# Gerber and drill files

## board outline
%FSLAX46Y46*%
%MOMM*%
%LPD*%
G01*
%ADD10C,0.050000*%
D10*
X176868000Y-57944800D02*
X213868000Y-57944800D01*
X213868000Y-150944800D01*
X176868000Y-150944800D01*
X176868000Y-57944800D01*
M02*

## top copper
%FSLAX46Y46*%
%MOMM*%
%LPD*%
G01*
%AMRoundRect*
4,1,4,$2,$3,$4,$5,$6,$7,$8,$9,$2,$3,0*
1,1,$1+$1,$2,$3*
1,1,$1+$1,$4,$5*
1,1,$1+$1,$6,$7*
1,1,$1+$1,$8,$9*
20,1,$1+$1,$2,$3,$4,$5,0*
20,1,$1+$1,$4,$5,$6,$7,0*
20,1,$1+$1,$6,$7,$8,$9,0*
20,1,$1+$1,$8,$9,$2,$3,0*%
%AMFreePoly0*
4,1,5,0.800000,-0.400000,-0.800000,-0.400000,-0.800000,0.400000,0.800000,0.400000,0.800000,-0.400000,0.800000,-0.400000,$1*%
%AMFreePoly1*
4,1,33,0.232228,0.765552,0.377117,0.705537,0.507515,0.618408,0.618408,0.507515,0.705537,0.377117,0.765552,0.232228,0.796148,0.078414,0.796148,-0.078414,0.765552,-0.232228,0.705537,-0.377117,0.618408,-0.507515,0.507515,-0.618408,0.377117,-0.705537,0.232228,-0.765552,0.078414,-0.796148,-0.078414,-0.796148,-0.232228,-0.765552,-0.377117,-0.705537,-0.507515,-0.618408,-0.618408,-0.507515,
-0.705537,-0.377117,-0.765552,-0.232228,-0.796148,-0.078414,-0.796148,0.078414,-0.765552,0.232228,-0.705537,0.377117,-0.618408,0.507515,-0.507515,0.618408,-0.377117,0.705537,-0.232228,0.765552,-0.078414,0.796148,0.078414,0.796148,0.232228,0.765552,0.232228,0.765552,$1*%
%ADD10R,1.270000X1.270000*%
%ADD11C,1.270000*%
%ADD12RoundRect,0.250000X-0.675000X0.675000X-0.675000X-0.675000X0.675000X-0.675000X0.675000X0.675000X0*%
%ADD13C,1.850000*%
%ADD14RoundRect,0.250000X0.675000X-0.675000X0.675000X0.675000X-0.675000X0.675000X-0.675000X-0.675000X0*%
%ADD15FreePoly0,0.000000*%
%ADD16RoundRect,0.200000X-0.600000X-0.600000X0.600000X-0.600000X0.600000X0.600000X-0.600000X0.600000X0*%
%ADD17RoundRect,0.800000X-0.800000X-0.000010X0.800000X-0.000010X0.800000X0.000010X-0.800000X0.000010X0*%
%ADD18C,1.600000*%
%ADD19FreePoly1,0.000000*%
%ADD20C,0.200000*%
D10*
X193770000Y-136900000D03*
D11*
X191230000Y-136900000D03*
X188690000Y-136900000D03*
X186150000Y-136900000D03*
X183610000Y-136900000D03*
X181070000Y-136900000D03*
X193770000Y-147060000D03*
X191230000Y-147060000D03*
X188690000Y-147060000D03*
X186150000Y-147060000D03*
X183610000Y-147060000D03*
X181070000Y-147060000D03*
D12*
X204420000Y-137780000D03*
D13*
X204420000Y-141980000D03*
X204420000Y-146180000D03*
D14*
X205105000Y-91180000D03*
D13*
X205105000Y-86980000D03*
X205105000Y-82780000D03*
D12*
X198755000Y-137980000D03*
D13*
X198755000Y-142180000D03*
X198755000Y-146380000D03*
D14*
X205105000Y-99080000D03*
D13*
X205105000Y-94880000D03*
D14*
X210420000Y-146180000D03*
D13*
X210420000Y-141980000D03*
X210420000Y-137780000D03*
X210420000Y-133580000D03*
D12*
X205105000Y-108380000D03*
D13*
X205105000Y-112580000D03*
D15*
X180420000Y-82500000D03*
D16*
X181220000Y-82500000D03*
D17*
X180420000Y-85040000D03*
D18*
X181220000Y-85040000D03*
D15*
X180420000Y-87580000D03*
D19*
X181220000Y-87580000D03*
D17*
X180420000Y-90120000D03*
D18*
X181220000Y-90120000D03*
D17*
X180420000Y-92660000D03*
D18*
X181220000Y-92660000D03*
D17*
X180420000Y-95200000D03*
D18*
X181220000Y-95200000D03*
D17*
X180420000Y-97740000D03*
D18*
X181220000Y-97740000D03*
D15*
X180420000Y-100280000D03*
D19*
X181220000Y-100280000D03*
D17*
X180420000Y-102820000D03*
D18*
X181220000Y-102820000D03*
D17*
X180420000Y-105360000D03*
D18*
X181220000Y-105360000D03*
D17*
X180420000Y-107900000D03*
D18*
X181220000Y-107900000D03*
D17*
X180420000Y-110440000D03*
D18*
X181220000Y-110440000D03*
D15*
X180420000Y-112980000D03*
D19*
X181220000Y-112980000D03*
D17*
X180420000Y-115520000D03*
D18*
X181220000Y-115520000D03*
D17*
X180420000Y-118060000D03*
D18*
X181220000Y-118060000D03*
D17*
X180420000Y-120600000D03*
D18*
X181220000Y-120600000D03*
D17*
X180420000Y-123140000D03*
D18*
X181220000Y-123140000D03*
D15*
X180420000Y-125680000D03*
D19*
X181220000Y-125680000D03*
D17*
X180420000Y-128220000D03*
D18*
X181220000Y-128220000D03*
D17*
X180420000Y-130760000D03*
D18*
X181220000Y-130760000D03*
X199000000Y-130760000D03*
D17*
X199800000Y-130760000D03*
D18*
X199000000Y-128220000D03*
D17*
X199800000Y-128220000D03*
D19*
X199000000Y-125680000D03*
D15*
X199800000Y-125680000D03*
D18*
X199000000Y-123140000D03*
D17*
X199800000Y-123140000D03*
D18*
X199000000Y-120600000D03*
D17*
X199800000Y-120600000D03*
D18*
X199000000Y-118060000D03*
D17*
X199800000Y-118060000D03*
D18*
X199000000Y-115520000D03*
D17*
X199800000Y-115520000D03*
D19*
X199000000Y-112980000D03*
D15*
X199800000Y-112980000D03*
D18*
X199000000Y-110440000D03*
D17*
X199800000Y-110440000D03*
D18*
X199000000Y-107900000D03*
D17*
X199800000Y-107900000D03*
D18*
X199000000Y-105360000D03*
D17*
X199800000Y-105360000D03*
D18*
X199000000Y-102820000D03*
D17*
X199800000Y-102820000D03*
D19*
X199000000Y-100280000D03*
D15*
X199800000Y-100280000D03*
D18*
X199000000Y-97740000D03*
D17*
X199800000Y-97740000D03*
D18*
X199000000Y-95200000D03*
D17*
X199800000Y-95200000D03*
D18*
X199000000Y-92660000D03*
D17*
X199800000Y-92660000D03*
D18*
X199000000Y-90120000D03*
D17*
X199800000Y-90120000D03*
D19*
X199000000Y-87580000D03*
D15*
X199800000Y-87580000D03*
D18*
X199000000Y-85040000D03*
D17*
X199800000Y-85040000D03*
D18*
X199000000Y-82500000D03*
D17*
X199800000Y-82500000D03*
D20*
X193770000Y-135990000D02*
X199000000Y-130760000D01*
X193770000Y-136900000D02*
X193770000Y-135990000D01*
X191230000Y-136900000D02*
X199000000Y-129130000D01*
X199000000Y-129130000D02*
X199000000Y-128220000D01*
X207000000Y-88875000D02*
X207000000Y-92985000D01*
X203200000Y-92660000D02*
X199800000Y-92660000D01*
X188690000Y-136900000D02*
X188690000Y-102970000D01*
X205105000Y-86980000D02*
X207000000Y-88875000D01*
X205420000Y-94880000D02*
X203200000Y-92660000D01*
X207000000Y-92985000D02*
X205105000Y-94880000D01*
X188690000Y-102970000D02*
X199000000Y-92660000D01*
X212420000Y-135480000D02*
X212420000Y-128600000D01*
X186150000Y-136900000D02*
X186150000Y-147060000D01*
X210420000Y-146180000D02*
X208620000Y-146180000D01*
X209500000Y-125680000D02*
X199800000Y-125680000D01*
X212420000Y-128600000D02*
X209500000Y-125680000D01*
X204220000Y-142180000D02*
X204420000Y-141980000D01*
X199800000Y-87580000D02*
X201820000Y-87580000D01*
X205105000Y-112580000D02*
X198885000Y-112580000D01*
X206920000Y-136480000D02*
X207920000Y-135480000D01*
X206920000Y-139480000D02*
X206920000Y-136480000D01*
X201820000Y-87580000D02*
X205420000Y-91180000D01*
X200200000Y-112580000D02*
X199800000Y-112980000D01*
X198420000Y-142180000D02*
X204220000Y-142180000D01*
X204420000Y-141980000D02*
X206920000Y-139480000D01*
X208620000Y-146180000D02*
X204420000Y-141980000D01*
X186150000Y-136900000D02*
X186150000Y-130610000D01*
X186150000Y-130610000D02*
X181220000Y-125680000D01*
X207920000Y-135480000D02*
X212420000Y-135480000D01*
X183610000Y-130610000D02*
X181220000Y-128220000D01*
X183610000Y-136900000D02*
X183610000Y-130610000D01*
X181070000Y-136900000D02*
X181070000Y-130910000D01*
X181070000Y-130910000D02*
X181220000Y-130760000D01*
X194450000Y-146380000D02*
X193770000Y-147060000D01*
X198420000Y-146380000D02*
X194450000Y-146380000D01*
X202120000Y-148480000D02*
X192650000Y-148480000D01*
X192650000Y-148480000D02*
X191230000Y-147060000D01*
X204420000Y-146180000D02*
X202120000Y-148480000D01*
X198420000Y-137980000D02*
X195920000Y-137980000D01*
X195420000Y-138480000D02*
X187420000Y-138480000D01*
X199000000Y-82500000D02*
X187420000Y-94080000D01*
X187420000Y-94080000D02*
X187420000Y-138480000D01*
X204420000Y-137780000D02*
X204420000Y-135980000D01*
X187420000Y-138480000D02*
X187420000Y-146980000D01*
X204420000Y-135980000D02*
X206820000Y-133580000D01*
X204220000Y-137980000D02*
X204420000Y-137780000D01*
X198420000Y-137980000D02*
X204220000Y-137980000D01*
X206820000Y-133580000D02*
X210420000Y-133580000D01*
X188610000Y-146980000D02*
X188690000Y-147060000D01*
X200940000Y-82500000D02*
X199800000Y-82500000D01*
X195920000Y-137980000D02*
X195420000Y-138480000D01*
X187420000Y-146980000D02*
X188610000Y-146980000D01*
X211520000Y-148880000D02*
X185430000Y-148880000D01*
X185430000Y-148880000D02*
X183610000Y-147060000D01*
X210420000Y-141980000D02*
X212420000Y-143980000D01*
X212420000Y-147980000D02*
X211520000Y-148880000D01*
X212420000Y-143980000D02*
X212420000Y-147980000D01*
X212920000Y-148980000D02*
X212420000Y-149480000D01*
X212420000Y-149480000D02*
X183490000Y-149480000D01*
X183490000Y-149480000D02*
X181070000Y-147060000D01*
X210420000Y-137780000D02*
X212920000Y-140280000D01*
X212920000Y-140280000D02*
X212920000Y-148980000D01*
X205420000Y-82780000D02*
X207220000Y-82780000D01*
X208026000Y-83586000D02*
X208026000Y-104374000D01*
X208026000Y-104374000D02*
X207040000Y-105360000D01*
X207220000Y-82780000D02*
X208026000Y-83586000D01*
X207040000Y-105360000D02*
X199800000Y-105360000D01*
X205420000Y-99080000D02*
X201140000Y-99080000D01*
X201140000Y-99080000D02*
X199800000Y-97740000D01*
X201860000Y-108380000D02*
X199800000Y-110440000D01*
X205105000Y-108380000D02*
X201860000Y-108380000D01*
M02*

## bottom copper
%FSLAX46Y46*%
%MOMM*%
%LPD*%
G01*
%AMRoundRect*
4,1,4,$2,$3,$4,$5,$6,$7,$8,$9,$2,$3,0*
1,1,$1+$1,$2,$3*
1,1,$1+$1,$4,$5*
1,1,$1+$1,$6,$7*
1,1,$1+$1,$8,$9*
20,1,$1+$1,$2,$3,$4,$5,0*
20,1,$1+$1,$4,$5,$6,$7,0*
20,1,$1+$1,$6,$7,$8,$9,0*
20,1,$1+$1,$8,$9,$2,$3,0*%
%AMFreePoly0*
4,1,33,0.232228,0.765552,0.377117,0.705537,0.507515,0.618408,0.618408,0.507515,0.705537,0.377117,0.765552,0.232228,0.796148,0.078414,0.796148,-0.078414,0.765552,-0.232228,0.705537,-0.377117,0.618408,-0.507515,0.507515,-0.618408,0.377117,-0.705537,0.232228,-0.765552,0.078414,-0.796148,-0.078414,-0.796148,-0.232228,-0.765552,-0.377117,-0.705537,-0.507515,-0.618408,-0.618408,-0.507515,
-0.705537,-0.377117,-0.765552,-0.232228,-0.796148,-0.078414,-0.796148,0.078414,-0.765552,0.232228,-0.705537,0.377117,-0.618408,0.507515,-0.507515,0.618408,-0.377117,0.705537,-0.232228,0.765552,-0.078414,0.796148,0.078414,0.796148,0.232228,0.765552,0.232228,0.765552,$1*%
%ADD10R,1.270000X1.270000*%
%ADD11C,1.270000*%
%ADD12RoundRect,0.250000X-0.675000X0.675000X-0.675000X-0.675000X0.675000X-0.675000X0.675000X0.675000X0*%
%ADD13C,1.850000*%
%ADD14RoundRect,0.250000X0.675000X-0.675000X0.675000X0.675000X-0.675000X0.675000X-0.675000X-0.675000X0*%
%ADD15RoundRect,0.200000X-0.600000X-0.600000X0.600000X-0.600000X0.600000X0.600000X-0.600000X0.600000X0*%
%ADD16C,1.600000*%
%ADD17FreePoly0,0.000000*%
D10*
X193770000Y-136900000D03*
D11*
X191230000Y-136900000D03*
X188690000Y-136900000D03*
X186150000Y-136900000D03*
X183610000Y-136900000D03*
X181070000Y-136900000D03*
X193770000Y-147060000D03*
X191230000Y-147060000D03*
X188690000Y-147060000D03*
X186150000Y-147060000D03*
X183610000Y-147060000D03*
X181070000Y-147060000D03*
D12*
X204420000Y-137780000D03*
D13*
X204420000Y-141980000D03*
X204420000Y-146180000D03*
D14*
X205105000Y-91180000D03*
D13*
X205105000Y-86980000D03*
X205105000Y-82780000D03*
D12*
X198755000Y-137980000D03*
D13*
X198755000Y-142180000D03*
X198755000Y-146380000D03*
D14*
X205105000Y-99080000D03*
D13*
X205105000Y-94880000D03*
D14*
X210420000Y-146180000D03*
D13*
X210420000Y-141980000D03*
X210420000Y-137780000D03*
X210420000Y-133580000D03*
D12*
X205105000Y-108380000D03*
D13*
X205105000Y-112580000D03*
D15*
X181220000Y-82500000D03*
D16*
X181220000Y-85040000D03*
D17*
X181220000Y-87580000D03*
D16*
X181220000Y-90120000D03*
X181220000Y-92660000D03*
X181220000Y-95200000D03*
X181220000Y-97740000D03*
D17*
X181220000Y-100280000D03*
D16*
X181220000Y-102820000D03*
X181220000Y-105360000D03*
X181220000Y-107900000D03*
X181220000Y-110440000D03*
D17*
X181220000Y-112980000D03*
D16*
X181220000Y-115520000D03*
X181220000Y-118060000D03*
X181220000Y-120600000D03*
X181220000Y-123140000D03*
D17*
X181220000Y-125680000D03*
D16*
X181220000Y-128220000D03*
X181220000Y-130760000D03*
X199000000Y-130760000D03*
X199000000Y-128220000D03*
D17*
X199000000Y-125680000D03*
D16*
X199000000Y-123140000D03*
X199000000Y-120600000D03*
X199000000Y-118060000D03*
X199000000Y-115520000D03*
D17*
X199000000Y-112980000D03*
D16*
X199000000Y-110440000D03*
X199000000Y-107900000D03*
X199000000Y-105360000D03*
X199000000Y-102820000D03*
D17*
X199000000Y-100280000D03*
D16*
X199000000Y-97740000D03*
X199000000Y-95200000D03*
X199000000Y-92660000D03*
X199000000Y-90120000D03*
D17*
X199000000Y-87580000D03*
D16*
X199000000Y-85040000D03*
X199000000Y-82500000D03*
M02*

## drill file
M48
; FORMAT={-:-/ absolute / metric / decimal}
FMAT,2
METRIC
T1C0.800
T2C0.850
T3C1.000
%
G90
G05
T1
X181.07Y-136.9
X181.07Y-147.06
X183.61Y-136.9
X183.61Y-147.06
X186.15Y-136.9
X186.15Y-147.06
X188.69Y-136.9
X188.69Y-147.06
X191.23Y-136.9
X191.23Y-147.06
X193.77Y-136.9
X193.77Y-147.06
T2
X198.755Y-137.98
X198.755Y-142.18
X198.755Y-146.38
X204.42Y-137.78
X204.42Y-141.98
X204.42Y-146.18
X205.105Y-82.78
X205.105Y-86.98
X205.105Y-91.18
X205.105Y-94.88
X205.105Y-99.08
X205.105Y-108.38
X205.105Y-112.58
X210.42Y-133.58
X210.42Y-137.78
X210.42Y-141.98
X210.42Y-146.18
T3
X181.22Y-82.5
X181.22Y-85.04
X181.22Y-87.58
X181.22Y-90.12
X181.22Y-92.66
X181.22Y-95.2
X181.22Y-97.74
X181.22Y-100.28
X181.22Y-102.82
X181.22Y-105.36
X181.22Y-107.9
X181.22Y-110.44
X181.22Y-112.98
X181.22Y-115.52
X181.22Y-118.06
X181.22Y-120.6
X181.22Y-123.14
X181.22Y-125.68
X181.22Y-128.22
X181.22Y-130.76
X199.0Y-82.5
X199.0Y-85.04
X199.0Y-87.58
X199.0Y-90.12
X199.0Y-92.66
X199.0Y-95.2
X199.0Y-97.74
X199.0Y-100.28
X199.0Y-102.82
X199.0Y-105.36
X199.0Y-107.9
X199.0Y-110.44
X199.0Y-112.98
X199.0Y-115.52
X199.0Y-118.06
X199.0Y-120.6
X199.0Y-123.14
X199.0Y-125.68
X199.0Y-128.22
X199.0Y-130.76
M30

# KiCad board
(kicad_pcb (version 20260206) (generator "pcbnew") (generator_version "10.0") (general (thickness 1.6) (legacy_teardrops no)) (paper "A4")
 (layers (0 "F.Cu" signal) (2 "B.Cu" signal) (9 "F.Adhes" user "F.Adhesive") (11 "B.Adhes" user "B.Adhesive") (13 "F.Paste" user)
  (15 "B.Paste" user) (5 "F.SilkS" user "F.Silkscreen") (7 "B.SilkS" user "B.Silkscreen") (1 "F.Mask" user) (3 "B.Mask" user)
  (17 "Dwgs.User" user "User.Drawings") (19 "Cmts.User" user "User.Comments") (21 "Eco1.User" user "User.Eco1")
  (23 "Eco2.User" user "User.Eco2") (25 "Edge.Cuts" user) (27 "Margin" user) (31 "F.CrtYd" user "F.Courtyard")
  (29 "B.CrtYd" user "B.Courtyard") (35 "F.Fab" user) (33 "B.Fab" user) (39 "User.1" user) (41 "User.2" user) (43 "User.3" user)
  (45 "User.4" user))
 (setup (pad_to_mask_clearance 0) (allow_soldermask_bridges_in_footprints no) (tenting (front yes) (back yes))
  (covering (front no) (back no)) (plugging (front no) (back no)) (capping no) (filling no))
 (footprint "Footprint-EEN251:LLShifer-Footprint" (layer "F.Cu") (at 187.42 141.98)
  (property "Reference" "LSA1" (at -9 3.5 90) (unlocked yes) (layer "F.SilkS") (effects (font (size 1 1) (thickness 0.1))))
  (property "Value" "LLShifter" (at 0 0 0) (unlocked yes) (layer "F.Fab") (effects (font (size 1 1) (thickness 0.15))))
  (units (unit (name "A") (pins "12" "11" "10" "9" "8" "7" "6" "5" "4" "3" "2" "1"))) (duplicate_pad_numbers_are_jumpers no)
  (pad "1" thru_hole rect (at 6.35 -5.08) (size 1.27 1.27) (drill 0.8) (layers "*.Cu" "*.Mask") (remove_unused_layers no) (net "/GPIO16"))
  (pad "2" thru_hole circle (at 3.81 -5.08) (size 1.27 1.27) (drill 0.8) (layers "*.Cu" "*.Mask") (remove_unused_layers no) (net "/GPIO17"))
  (pad "3" thru_hole circle (at 1.27 -5.08) (size 1.27 1.27) (drill 0.8) (layers "*.Cu" "*.Mask") (remove_unused_layers no) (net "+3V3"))
  (pad "4" thru_hole circle (at -1.27 -5.08) (size 1.27 1.27) (drill 0.8) (layers "*.Cu" "*.Mask") (remove_unused_layers no) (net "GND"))
  (pad "5" thru_hole circle (at -3.81 -5.08) (size 1.27 1.27) (drill 0.8) (layers "*.Cu" "*.Mask") (remove_unused_layers no) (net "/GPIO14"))
  (pad "6" thru_hole circle (at -6.35 -5.08) (size 1.27 1.27) (drill 0.8) (layers "*.Cu" "*.Mask") (remove_unused_layers no) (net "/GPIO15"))
  (pad "7" thru_hole circle (at 6.35 5.08) (size 1.27 1.27) (drill 0.8) (layers "*.Cu" "*.Mask") (remove_unused_layers no) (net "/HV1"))
  (pad "8" thru_hole circle (at 3.81 5.08) (size 1.27 1.27) (drill 0.8) (layers "*.Cu" "*.Mask") (remove_unused_layers no) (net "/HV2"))
  (pad "9" thru_hole circle (at 1.27 5.08) (size 1.27 1.27) (drill 0.8) (layers "*.Cu" "*.Mask") (remove_unused_layers no) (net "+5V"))
  (pad "10" thru_hole circle (at -1.27 5.08) (size 1.27 1.27) (drill 0.8) (layers "*.Cu" "*.Mask") (remove_unused_layers no) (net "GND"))
  (pad "11" thru_hole circle (at -3.81 5.08) (size 1.27 1.27) (drill 0.8) (layers "*.Cu" "*.Mask") (remove_unused_layers no) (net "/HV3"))
  (pad "12" thru_hole circle (at -6.35 5.08) (size 1.27 1.27) (drill 0.8) (layers "*.Cu" "*.Mask") (remove_unused_layers no) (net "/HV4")))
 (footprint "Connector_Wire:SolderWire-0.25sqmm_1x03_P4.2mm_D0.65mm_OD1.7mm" (layer "F.Cu") (at 204.42 137.78 -90)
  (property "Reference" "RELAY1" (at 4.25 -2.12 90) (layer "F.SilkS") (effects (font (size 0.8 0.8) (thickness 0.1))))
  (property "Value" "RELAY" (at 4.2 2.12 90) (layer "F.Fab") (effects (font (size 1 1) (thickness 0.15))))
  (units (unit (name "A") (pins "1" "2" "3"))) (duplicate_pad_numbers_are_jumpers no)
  (pad "1" thru_hole roundrect (at 0 0 270) (size 1.85 1.85) (drill 0.85) (layers "*.Cu" "*.Mask") (remove_unused_layers no)
   (roundrect_rratio 0.135135) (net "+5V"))
  (pad "2" thru_hole circle (at 4.2 0 270) (size 1.85 1.85) (drill 0.85) (layers "*.Cu" "*.Mask") (remove_unused_layers no) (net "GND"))
  (pad "3" thru_hole circle (at 8.4 0 270) (size 1.85 1.85) (drill 0.85) (layers "*.Cu" "*.Mask") (remove_unused_layers no) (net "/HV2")))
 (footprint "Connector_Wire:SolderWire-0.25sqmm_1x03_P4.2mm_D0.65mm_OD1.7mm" (layer "F.Cu") (at 205.105 91.18 90)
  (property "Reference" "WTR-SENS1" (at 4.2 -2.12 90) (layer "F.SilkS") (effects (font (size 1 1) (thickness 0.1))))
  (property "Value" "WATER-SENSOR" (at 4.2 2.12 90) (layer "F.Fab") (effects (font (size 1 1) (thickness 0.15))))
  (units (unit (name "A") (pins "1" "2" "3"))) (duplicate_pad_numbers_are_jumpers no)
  (pad "1" thru_hole roundrect (at 0 0 90) (size 1.85 1.85) (drill 0.85) (layers "*.Cu" "*.Mask") (remove_unused_layers no)
   (roundrect_rratio 0.135135) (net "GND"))
  (pad "2" thru_hole circle (at 4.2 0 90) (size 1.85 1.85) (drill 0.85) (layers "*.Cu" "*.Mask") (remove_unused_layers no) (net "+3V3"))
  (pad "3" thru_hole circle (at 8.4 0 90) (size 1.85 1.85) (drill 0.85) (layers "*.Cu" "*.Mask") (remove_unused_layers no) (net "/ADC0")))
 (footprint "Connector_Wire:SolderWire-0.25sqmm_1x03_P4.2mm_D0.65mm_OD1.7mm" (layer "F.Cu") (at 198.755 137.98 -90)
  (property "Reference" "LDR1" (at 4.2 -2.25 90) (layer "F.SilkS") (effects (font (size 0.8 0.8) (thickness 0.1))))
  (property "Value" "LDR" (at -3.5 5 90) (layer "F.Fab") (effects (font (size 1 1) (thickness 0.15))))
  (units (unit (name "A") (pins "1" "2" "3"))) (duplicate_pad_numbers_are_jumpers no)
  (pad "1" thru_hole roundrect (at 0 0 270) (size 1.85 1.85) (drill 0.85) (layers "*.Cu" "*.Mask") (remove_unused_layers no)
   (roundrect_rratio 0.135135) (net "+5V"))
  (pad "2" thru_hole circle (at 4.2 0 270) (size 1.85 1.85) (drill 0.85) (layers "*.Cu" "*.Mask") (remove_unused_layers no) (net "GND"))
  (pad "3" thru_hole circle (at 8.4 0 270) (size 1.85 1.85) (drill 0.85) (layers "*.Cu" "*.Mask") (remove_unused_layers no) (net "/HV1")))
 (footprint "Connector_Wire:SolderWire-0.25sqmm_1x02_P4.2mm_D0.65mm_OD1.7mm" (layer "F.Cu") (at 205.105 99.08 90)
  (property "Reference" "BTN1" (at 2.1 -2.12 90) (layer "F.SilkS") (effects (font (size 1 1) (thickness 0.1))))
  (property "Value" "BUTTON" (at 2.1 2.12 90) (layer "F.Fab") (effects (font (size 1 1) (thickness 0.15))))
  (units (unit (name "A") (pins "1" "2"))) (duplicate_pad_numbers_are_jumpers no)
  (pad "1" thru_hole roundrect (at 0 0 90) (size 1.85 1.85) (drill 0.85) (layers "*.Cu" "*.Mask") (remove_unused_layers no)
   (roundrect_rratio 0.135135) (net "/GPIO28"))
  (pad "2" thru_hole circle (at 4.2 0 90) (size 1.85 1.85) (drill 0.85) (layers "*.Cu" "*.Mask") (remove_unused_layers no) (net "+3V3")))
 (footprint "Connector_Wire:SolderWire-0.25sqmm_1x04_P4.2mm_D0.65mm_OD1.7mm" (layer "F.Cu") (at 210.42 146.18 90)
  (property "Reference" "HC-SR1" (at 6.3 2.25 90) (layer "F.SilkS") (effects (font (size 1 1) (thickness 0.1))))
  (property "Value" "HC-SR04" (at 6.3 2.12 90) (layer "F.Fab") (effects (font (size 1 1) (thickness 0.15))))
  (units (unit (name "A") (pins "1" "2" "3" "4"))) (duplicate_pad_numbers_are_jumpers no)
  (pad "1" thru_hole roundrect (at 0 0 90) (size 1.85 1.85) (drill 0.85) (layers "*.Cu" "*.Mask") (remove_unused_layers no)
   (roundrect_rratio 0.135135) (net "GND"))
  (pad "2" thru_hole circle (at 4.2 0 90) (size 1.85 1.85) (drill 0.85) (layers "*.Cu" "*.Mask") (remove_unused_layers no) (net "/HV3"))
  (pad "3" thru_hole circle (at 8.4 0 90) (size 1.85 1.85) (drill 0.85) (layers "*.Cu" "*.Mask") (remove_unused_layers no) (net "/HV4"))
  (pad "4" thru_hole circle (at 12.6 0 90) (size 1.85 1.85) (drill 0.85) (layers "*.Cu" "*.Mask") (remove_unused_layers no) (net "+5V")))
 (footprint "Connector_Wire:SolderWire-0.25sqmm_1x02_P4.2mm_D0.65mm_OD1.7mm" (layer "F.Cu") (at 205.105 108.38 -90)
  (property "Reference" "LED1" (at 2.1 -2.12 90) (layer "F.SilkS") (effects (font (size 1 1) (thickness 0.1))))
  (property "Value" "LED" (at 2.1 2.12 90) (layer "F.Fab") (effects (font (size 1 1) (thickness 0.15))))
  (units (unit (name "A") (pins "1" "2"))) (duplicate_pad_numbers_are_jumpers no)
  (pad "1" thru_hole roundrect (at 0 0 270) (size 1.85 1.85) (drill 0.85) (layers "*.Cu" "*.Mask") (remove_unused_layers no)
   (roundrect_rratio 0.135135) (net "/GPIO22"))
  (pad "2" thru_hole circle (at 4.2 0 270) (size 1.85 1.85) (drill 0.85) (layers "*.Cu" "*.Mask") (remove_unused_layers no) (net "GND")))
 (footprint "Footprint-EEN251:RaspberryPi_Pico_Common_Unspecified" (layer "F.Cu") (at 190.11 106.63)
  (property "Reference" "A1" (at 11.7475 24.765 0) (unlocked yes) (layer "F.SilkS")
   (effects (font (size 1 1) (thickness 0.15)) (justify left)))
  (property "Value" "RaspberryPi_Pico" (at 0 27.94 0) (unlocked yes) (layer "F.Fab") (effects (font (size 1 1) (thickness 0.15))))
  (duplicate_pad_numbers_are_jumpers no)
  (pad "1" smd custom (at -9.69 -24.13) (size 1.6 0.8) (layers "F.Cu" "F.Mask") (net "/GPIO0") (options (clearance outline) (anchor rect))
   (primitives))
  (pad "1" thru_hole roundrect (at -8.89 -24.13) (size 1.6 1.6) (drill 1) (layers "*.Cu" "*.Mask") (remove_unused_layers no)
   (roundrect_rratio 0.125) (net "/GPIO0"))
  (pad "2" smd roundrect (at -9.69 -21.59) (size 3.2 1.6) (layers "F.Cu" "F.Mask") (roundrect_rratio 0.5) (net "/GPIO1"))
  (pad "2" thru_hole circle (at -8.89 -21.59) (size 1.6 1.6) (drill 1) (layers "*.Cu" "*.Mask") (remove_unused_layers no) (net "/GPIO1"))
  (pad "3" smd custom (at -9.69 -19.05) (size 1.6 0.8) (layers "F.Cu" "F.Mask") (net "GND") (options (clearance outline) (anchor rect))
   (primitives))
  (pad "3" thru_hole custom (at -8.89 -19.05) (size 1.6 1.6) (drill 1) (layers "*.Cu" "*.Mask") (remove_unused_layers no) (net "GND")
   (options (clearance outline) (anchor circle)) (primitives))
  (pad "4" smd roundrect (at -9.69 -16.51) (size 3.2 1.6) (layers "F.Cu" "F.Mask") (roundrect_rratio 0.5)
   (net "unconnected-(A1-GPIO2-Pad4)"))
  (pad "4" thru_hole circle (at -8.89 -16.51) (size 1.6 1.6) (drill 1) (layers "*.Cu" "*.Mask") (remove_unused_layers no)
   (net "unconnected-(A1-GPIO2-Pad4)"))
  (pad "5" smd roundrect (at -9.69 -13.97) (size 3.2 1.6) (layers "F.Cu" "F.Mask") (roundrect_rratio 0.5)
   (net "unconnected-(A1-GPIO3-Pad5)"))
  (pad "5" thru_hole circle (at -8.89 -13.97) (size 1.6 1.6) (drill 1) (layers "*.Cu" "*.Mask") (remove_unused_layers no)
   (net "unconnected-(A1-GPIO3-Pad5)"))
  (pad "6" smd roundrect (at -9.69 -11.43) (size 3.2 1.6) (layers "F.Cu" "F.Mask") (roundrect_rratio 0.5)
   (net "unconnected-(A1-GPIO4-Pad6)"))
  (pad "6" thru_hole circle (at -8.89 -11.43) (size 1.6 1.6) (drill 1) (layers "*.Cu" "*.Mask") (remove_unused_layers no)
   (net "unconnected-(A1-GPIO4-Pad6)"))
  (pad "7" smd roundrect (at -9.69 -8.89) (size 3.2 1.6) (layers "F.Cu" "F.Mask") (roundrect_rratio 0.5) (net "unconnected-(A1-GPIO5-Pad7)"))
  (pad "7" thru_hole circle (at -8.89 -8.89) (size 1.6 1.6) (drill 1) (layers "*.Cu" "*.Mask") (remove_unused_layers no)
   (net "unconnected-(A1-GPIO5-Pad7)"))
  (pad "8" smd custom (at -9.69 -6.35) (size 1.6 0.8) (layers "F.Cu" "F.Mask") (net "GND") (options (clearance outline) (anchor rect))
   (primitives))
  (pad "8" thru_hole custom (at -8.89 -6.35) (size 1.6 1.6) (drill 1) (layers "*.Cu" "*.Mask") (remove_unused_layers no) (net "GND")
   (options (clearance outline) (anchor circle)) (primitives))
  (pad "9" smd roundrect (at -9.69 -3.81) (size 3.2 1.6) (layers "F.Cu" "F.Mask") (roundrect_rratio 0.5) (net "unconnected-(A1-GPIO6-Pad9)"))
  (pad "9" thru_hole circle (at -8.89 -3.81) (size 1.6 1.6) (drill 1) (layers "*.Cu" "*.Mask") (remove_unused_layers no)
   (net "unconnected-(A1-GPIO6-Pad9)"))
  (pad "10" smd roundrect (at -9.69 -1.27) (size 3.2 1.6) (layers "F.Cu" "F.Mask") (roundrect_rratio 0.5)
   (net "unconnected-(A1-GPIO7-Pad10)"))
  (pad "10" thru_hole circle (at -8.89 -1.27) (size 1.6 1.6) (drill 1) (layers "*.Cu" "*.Mask") (remove_unused_layers no)
   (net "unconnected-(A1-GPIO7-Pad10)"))
  (pad "11" smd roundrect (at -9.69 1.27) (size 3.2 1.6) (layers "F.Cu" "F.Mask") (roundrect_rratio 0.5)
   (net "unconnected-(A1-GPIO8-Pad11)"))
  (pad "11" thru_hole circle (at -8.89 1.27) (size 1.6 1.6) (drill 1) (layers "*.Cu" "*.Mask") (remove_unused_layers no)
   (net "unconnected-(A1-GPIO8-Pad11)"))
  (pad "12" smd roundrect (at -9.69 3.81) (size 3.2 1.6) (layers "F.Cu" "F.Mask") (roundrect_rratio 0.5)
   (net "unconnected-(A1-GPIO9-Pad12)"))
  (pad "12" thru_hole circle (at -8.89 3.81) (size 1.6 1.6) (drill 1) (layers "*.Cu" "*.Mask") (remove_unused_layers no)
   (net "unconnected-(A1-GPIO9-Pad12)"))
  (pad "13" smd custom (at -9.69 6.35) (size 1.6 0.8) (layers "F.Cu" "F.Mask") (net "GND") (options (clearance outline) (anchor rect))
   (primitives))
  (pad "13" thru_hole custom (at -8.89 6.35) (size 1.6 1.6) (drill 1) (layers "*.Cu" "*.Mask") (remove_unused_layers no) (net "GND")
   (options (clearance outline) (anchor circle)) (primitives))
  (pad "14" smd roundrect (at -9.69 8.89) (size 3.2 1.6) (layers "F.Cu" "F.Mask") (roundrect_rratio 0.5)
   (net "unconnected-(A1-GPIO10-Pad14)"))
  (pad "14" thru_hole circle (at -8.89 8.89) (size 1.6 1.6) (drill 1) (layers "*.Cu" "*.Mask") (remove_unused_layers no)
   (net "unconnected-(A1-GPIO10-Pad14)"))
  (pad "15" smd roundrect (at -9.69 11.43) (size 3.2 1.6) (layers "F.Cu" "F.Mask") (roundrect_rratio 0.5)
   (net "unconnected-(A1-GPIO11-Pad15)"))
  (pad "15" thru_hole circle (at -8.89 11.43) (size 1.6 1.6) (drill 1) (layers "*.Cu" "*.Mask") (remove_unused_layers no)
   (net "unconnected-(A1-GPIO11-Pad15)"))
  (pad "16" smd roundrect (at -9.69 13.97) (size 3.2 1.6) (layers "F.Cu" "F.Mask") (roundrect_rratio 0.5)
   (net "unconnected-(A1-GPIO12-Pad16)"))
  (pad "16" thru_hole circle (at -8.89 13.97) (size 1.6 1.6) (drill 1) (layers "*.Cu" "*.Mask") (remove_unused_layers no)
   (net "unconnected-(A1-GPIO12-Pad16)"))
  (pad "17" smd roundrect (at -9.69 16.51) (size 3.2 1.6) (layers "F.Cu" "F.Mask") (roundrect_rratio 0.5)
   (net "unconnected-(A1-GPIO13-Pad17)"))
  (pad "17" thru_hole circle (at -8.89 16.51) (size 1.6 1.6) (drill 1) (layers "*.Cu" "*.Mask") (remove_unused_layers no)
   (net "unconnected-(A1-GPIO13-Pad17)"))
  (pad "18" smd custom (at -9.69 19.05) (size 1.6 0.8) (layers "F.Cu" "F.Mask") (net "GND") (options (clearance outline) (anchor rect))
   (primitives))
  (pad "18" thru_hole custom (at -8.89 19.05) (size 1.6 1.6) (drill 1) (layers "*.Cu" "*.Mask") (remove_unused_layers no) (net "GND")
   (options (clearance outline) (anchor circle)) (primitives))
  (pad "19" smd roundrect (at -9.69 21.59) (size 3.2 1.6) (layers "F.Cu" "F.Mask") (roundrect_rratio 0.5) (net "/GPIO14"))
  (pad "19" thru_hole circle (at -8.89 21.59) (size 1.6 1.6) (drill 1) (layers "*.Cu" "*.Mask") (remove_unused_layers no) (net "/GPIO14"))
  (pad "20" smd roundrect (at -9.69 24.13) (size 3.2 1.6) (layers "F.Cu" "F.Mask") (roundrect_rratio 0.5) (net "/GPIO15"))
  (pad "20" thru_hole circle (at -8.89 24.13) (size 1.6 1.6) (drill 1) (layers "*.Cu" "*.Mask") (remove_unused_layers no) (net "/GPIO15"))
  (pad "21" thru_hole circle (at 8.89 24.13) (size 1.6 1.6) (drill 1) (layers "*.Cu" "*.Mask") (remove_unused_layers no) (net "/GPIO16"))
  (pad "21" smd roundrect (at 9.69 24.13) (size 3.2 1.6) (layers "F.Cu" "F.Mask") (roundrect_rratio 0.5) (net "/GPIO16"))
  (pad "22" thru_hole circle (at 8.89 21.59) (size 1.6 1.6) (drill 1) (layers "*.Cu" "*.Mask") (remove_unused_layers no) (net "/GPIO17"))
  (pad "22" smd roundrect (at 9.69 21.59) (size 3.2 1.6) (layers "F.Cu" "F.Mask") (roundrect_rratio 0.5) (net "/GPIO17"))
  (pad "23" thru_hole custom (at 8.89 19.05) (size 1.6 1.6) (drill 1) (layers "*.Cu" "*.Mask") (remove_unused_layers no) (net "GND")
   (options (clearance outline) (anchor circle)) (primitives))
  (pad "23" smd custom (at 9.69 19.05) (size 1.6 0.8) (layers "F.Cu" "F.Mask") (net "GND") (options (clearance outline) (anchor rect))
   (primitives))
  (pad "24" thru_hole circle (at 8.89 16.51) (size 1.6 1.6) (drill 1) (layers "*.Cu" "*.Mask") (remove_unused_layers no) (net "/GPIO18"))
  (pad "24" smd roundrect (at 9.69 16.51) (size 3.2 1.6) (layers "F.Cu" "F.Mask") (roundrect_rratio 0.5) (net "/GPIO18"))
  (pad "25" thru_hole circle (at 8.89 13.97) (size 1.6 1.6) (drill 1) (layers "*.Cu" "*.Mask") (remove_unused_layers no) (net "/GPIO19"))
  (pad "25" smd roundrect (at 9.69 13.97) (size 3.2 1.6) (layers "F.Cu" "F.Mask") (roundrect_rratio 0.5) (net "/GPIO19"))
  (pad "26" thru_hole circle (at 8.89 11.43) (size 1.6 1.6) (drill 1) (layers "*.Cu" "*.Mask") (remove_unused_layers no)
   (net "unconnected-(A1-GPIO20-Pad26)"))
  (pad "26" smd roundrect (at 9.69 11.43) (size 3.2 1.6) (layers "F.Cu" "F.Mask") (roundrect_rratio 0.5)
   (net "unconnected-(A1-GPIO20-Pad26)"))
  (pad "27" thru_hole circle (at 8.89 8.89) (size 1.6 1.6) (drill 1) (layers "*.Cu" "*.Mask") (remove_unused_layers no)
   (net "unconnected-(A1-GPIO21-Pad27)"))
  (pad "27" smd roundrect (at 9.69 8.89) (size 3.2 1.6) (layers "F.Cu" "F.Mask") (roundrect_rratio 0.5)
   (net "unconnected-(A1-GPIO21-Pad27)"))
  (pad "28" thru_hole custom (at 8.89 6.35) (size 1.6 1.6) (drill 1) (layers "*.Cu" "*.Mask") (remove_unused_layers no) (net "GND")
   (options (clearance outline) (anchor circle)) (primitives))
  (pad "28" smd custom (at 9.69 6.35) (size 1.6 0.8) (layers "F.Cu" "F.Mask") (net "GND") (options (clearance outline) (anchor rect))
   (primitives))
  (pad "29" thru_hole circle (at 8.89 3.81) (size 1.6 1.6) (drill 1) (layers "*.Cu" "*.Mask") (remove_unused_layers no) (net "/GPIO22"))
  (pad "29" smd roundrect (at 9.69 3.81) (size 3.2 1.6) (layers "F.Cu" "F.Mask") (roundrect_rratio 0.5) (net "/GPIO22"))
  (pad "30" thru_hole circle (at 8.89 1.27) (size 1.6 1.6) (drill 1) (layers "*.Cu" "*.Mask") (remove_unused_layers no)
   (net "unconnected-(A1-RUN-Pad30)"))
  (pad "30" smd roundrect (at 9.69 1.27) (size 3.2 1.6) (layers "F.Cu" "F.Mask") (roundrect_rratio 0.5) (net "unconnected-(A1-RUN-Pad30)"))
  (pad "31" thru_hole circle (at 8.89 -1.27) (size 1.6 1.6) (drill 1) (layers "*.Cu" "*.Mask") (remove_unused_layers no) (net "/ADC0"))
  (pad "31" smd roundrect (at 9.69 -1.27) (size 3.2 1.6) (layers "F.Cu" "F.Mask") (roundrect_rratio 0.5) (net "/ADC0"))
  (pad "32" thru_hole circle (at 8.89 -3.81) (size 1.6 1.6) (drill 1) (layers "*.Cu" "*.Mask") (remove_unused_layers no) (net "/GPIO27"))
  (pad "32" smd roundrect (at 9.69 -3.81) (size 3.2 1.6) (layers "F.Cu" "F.Mask") (roundrect_rratio 0.5) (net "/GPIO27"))
  (pad "33" thru_hole custom (at 8.89 -6.35) (size 1.6 1.6) (drill 1) (layers "*.Cu" "*.Mask") (remove_unused_layers no)
   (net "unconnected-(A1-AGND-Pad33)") (options (clearance outline) (anchor circle)) (primitives))
  (pad "33" smd custom (at 9.69 -6.35) (size 1.6 0.8) (layers "F.Cu" "F.Mask") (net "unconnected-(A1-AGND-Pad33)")
   (options (clearance outline) (anchor rect)) (primitives))
  (pad "34" thru_hole circle (at 8.89 -8.89) (size 1.6 1.6) (drill 1) (layers "*.Cu" "*.Mask") (remove_unused_layers no) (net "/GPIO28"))
  (pad "34" smd roundrect (at 9.69 -8.89) (size 3.2 1.6) (layers "F.Cu" "F.Mask") (roundrect_rratio 0.5) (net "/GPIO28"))
  (pad "35" thru_hole circle (at 8.89 -11.43) (size 1.6 1.6) (drill 1) (layers "*.Cu" "*.Mask") (remove_unused_layers no)
   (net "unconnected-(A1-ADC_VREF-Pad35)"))
  (pad "35" smd roundrect (at 9.69 -11.43) (size 3.2 1.6) (layers "F.Cu" "F.Mask") (roundrect_rratio 0.5)
   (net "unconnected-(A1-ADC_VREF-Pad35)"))
  (pad "36" thru_hole circle (at 8.89 -13.97) (size 1.6 1.6) (drill 1) (layers "*.Cu" "*.Mask") (remove_unused_layers no) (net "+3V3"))
  (pad "36" smd roundrect (at 9.69 -13.97) (size 3.2 1.6) (layers "F.Cu" "F.Mask") (roundrect_rratio 0.5) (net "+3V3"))
  (pad "37" thru_hole circle (at 8.89 -16.51) (size 1.6 1.6) (drill 1) (layers "*.Cu" "*.Mask") (remove_unused_layers no)
   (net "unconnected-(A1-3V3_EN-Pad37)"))
  (pad "37" smd roundrect (at 9.69 -16.51) (size 3.2 1.6) (layers "F.Cu" "F.Mask") (roundrect_rratio 0.5)
   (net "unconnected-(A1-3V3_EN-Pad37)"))
  (pad "38" thru_hole custom (at 8.89 -19.05) (size 1.6 1.6) (drill 1) (layers "*.Cu" "*.Mask") (remove_unused_layers no) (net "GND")
   (options (clearance outline) (anchor circle)) (primitives))
  (pad "38" smd custom (at 9.69 -19.05) (size 1.6 0.8) (layers "F.Cu" "F.Mask") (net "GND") (options (clearance outline) (anchor rect))
   (primitives))
  (pad "39" thru_hole circle (at 8.89 -21.59) (size 1.6 1.6) (drill 1) (layers "*.Cu" "*.Mask") (remove_unused_layers no)
   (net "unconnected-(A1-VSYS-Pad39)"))
  (pad "39" smd roundrect (at 9.69 -21.59) (size 3.2 1.6) (layers "F.Cu" "F.Mask") (roundrect_rratio 0.5)
   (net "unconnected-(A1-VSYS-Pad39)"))
  (pad "40" thru_hole circle (at 8.89 -24.13) (size 1.6 1.6) (drill 1) (layers "*.Cu" "*.Mask") (remove_unused_layers no) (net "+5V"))
  (pad "40" smd roundrect (at 9.69 -24.13) (size 3.2 1.6) (layers "F.Cu" "F.Mask") (roundrect_rratio 0.5) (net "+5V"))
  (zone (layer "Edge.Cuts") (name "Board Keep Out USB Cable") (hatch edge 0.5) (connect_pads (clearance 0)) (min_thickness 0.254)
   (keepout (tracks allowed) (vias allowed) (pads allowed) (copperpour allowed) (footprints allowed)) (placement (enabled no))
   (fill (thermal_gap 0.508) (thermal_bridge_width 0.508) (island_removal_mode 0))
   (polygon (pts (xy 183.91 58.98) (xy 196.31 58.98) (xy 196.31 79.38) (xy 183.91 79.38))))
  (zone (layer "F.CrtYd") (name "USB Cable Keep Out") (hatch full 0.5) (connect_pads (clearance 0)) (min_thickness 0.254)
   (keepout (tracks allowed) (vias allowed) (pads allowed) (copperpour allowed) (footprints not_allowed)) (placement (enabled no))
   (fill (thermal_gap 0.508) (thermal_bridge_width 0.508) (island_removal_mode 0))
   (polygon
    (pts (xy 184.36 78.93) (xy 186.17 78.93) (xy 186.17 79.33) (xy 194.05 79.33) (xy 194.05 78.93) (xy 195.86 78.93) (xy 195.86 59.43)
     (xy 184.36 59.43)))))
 (gr_rect (start 176.868 57.9448) (end 213.868 150.9448) (stroke (width 0.05) (type default)) (fill no) (layer "Edge.Cuts"))
 (segment (start 193.77 135.99) (end 199 130.76) (width 0.2) (layer "F.Cu") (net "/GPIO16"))
 (segment (start 193.77 136.9) (end 193.77 135.99) (width 0.2) (layer "F.Cu") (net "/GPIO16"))
 (segment (start 191.23 136.9) (end 199 129.13) (width 0.2) (layer "F.Cu") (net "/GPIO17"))
 (segment (start 199 129.13) (end 199 128.22) (width 0.2) (layer "F.Cu") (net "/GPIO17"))
 (segment (start 207 88.875) (end 207 92.985) (width 0.2) (layer "F.Cu") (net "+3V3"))
 (segment (start 203.2 92.66) (end 199.8 92.66) (width 0.2) (layer "F.Cu") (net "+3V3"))
 (segment (start 188.69 136.9) (end 188.69 102.97) (width 0.2) (layer "F.Cu") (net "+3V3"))
 (segment (start 205.105 86.98) (end 207 88.875) (width 0.2) (layer "F.Cu") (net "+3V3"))
 (segment (start 205.42 94.88) (end 203.2 92.66) (width 0.2) (layer "F.Cu") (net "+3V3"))
 (segment (start 207 92.985) (end 205.105 94.88) (width 0.2) (layer "F.Cu") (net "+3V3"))
 (segment (start 188.69 102.97) (end 199 92.66) (width 0.2) (layer "F.Cu") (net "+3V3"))
 (segment (start 212.42 135.48) (end 212.42 128.6) (width 0.2) (layer "F.Cu") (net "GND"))
 (segment (start 186.15 136.9) (end 186.15 147.06) (width 0.2) (layer "F.Cu") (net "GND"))
 (segment (start 210.42 146.18) (end 208.62 146.18) (width 0.2) (layer "F.Cu") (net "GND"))
 (segment (start 209.5 125.68) (end 199.8 125.68) (width 0.2) (layer "F.Cu") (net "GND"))
 (segment (start 212.42 128.6) (end 209.5 125.68) (width 0.2) (layer "F.Cu") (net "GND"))
 (segment (start 204.22 142.18) (end 204.42 141.98) (width 0.2) (layer "F.Cu") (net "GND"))
 (segment (start 199.8 87.58) (end 201.82 87.58) (width 0.2) (layer "F.Cu") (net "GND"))
 (segment (start 205.105 112.58) (end 198.885 112.58) (width 0.2) (layer "F.Cu") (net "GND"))
 (segment (start 206.92 136.48) (end 207.92 135.48) (width 0.2) (layer "F.Cu") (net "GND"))
 (segment (start 206.92 139.48) (end 206.92 136.48) (width 0.2) (layer "F.Cu") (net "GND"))
 (segment (start 201.82 87.58) (end 205.42 91.18) (width 0.2) (layer "F.Cu") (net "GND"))
 (segment (start 200.2 112.58) (end 199.8 112.98) (width 0.2) (layer "F.Cu") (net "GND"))
 (segment (start 198.42 142.18) (end 204.22 142.18) (width 0.2) (layer "F.Cu") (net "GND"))
 (segment (start 204.42 141.98) (end 206.92 139.48) (width 0.2) (layer "F.Cu") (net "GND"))
 (segment (start 208.62 146.18) (end 204.42 141.98) (width 0.2) (layer "F.Cu") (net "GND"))
 (segment (start 186.15 136.9) (end 186.15 130.61) (width 0.2) (layer "F.Cu") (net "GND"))
 (segment (start 186.15 130.61) (end 181.22 125.68) (width 0.2) (layer "F.Cu") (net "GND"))
 (segment (start 207.92 135.48) (end 212.42 135.48) (width 0.2) (layer "F.Cu") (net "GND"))
 (segment (start 183.61 130.61) (end 181.22 128.22) (width 0.2) (layer "F.Cu") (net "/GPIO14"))
 (segment (start 183.61 136.9) (end 183.61 130.61) (width 0.2) (layer "F.Cu") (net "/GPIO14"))
 (segment (start 181.07 136.9) (end 181.07 130.91) (width 0.2) (layer "F.Cu") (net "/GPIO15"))
 (segment (start 181.07 130.91) (end 181.22 130.76) (width 0.2) (layer "F.Cu") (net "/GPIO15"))
 (segment (start 194.45 146.38) (end 193.77 147.06) (width 0.2) (layer "F.Cu") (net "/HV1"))
 (segment (start 198.42 146.38) (end 194.45 146.38) (width 0.2) (layer "F.Cu") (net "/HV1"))
 (segment (start 202.12 148.48) (end 192.65 148.48) (width 0.2) (layer "F.Cu") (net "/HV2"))
 (segment (start 192.65 148.48) (end 191.23 147.06) (width 0.2) (layer "F.Cu") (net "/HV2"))
 (segment (start 204.42 146.18) (end 202.12 148.48) (width 0.2) (layer "F.Cu") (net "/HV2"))
 (segment (start 198.42 137.98) (end 195.92 137.98) (width 0.2) (layer "F.Cu") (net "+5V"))
 (segment (start 195.42 138.48) (end 187.42 138.48) (width 0.2) (layer "F.Cu") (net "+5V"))
 (segment (start 199 82.5) (end 187.42 94.08) (width 0.2) (layer "F.Cu") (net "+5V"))
 (segment (start 187.42 94.08) (end 187.42 138.48) (width 0.2) (layer "F.Cu") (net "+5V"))
 (segment (start 204.42 137.78) (end 204.42 135.98) (width 0.2) (layer "F.Cu") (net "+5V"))
 (segment (start 187.42 138.48) (end 187.42 146.98) (width 0.2) (layer "F.Cu") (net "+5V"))
 (segment (start 204.42 135.98) (end 206.82 133.58) (width 0.2) (layer "F.Cu") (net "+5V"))
 (segment (start 204.22 137.98) (end 204.42 137.78) (width 0.2) (layer "F.Cu") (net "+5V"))
 (segment (start 198.42 137.98) (end 204.22 137.98) (width 0.2) (layer "F.Cu") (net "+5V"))
 (segment (start 206.82 133.58) (end 210.42 133.58) (width 0.2) (layer "F.Cu") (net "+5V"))
 (segment (start 188.61 146.98) (end 188.69 147.06) (width 0.2) (layer "F.Cu") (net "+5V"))
 (segment (start 200.94 82.5) (end 199.8 82.5) (width 0.2) (layer "F.Cu") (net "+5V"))
 (segment (start 195.92 137.98) (end 195.42 138.48) (width 0.2) (layer "F.Cu") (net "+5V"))
 (segment (start 187.42 146.98) (end 188.61 146.98) (width 0.2) (layer "F.Cu") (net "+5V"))
 (segment (start 211.52 148.88) (end 185.43 148.88) (width 0.2) (layer "F.Cu") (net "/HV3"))
 (segment (start 185.43 148.88) (end 183.61 147.06) (width 0.2) (layer "F.Cu") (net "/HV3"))
 (segment (start 210.42 141.98) (end 212.42 143.98) (width 0.2) (layer "F.Cu") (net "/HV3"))
 (segment (start 212.42 147.98) (end 211.52 148.88) (width 0.2) (layer "F.Cu") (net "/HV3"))
 (segment (start 212.42 143.98) (end 212.42 147.98) (width 0.2) (layer "F.Cu") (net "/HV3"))
 (segment (start 212.92 148.98) (end 212.42 149.48) (width 0.2) (layer "F.Cu") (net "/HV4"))
 (segment (start 212.42 149.48) (end 183.49 149.48) (width 0.2) (layer "F.Cu") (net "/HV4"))
 (segment (start 183.49 149.48) (end 181.07 147.06) (width 0.2) (layer "F.Cu") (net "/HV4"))
 (segment (start 210.42 137.78) (end 212.92 140.28) (width 0.2) (layer "F.Cu") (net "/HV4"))
 (segment (start 212.92 140.28) (end 212.92 148.98) (width 0.2) (layer "F.Cu") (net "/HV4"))
 (segment (start 205.42 82.78) (end 207.22 82.78) (width 0.2) (layer "F.Cu") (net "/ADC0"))
 (segment (start 208.026 83.586) (end 208.026 104.374) (width 0.2) (layer "F.Cu") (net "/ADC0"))
 (segment (start 208.026 104.374) (end 207.04 105.36) (width 0.2) (layer "F.Cu") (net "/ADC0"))
 (segment (start 207.22 82.78) (end 208.026 83.586) (width 0.2) (layer "F.Cu") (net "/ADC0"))
 (segment (start 207.04 105.36) (end 199.8 105.36) (width 0.2) (layer "F.Cu") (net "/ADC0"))
 (segment (start 205.42 99.08) (end 201.14 99.08) (width 0.2) (layer "F.Cu") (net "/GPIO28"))
 (segment (start 201.14 99.08) (end 199.8 97.74) (width 0.2) (layer "F.Cu") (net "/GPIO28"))
 (segment (start 201.86 108.38) (end 199.8 110.44) (width 0.2) (layer "F.Cu") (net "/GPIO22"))
 (segment (start 205.105 108.38) (end 201.86 108.38) (width 0.2) (layer "F.Cu") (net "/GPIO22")))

